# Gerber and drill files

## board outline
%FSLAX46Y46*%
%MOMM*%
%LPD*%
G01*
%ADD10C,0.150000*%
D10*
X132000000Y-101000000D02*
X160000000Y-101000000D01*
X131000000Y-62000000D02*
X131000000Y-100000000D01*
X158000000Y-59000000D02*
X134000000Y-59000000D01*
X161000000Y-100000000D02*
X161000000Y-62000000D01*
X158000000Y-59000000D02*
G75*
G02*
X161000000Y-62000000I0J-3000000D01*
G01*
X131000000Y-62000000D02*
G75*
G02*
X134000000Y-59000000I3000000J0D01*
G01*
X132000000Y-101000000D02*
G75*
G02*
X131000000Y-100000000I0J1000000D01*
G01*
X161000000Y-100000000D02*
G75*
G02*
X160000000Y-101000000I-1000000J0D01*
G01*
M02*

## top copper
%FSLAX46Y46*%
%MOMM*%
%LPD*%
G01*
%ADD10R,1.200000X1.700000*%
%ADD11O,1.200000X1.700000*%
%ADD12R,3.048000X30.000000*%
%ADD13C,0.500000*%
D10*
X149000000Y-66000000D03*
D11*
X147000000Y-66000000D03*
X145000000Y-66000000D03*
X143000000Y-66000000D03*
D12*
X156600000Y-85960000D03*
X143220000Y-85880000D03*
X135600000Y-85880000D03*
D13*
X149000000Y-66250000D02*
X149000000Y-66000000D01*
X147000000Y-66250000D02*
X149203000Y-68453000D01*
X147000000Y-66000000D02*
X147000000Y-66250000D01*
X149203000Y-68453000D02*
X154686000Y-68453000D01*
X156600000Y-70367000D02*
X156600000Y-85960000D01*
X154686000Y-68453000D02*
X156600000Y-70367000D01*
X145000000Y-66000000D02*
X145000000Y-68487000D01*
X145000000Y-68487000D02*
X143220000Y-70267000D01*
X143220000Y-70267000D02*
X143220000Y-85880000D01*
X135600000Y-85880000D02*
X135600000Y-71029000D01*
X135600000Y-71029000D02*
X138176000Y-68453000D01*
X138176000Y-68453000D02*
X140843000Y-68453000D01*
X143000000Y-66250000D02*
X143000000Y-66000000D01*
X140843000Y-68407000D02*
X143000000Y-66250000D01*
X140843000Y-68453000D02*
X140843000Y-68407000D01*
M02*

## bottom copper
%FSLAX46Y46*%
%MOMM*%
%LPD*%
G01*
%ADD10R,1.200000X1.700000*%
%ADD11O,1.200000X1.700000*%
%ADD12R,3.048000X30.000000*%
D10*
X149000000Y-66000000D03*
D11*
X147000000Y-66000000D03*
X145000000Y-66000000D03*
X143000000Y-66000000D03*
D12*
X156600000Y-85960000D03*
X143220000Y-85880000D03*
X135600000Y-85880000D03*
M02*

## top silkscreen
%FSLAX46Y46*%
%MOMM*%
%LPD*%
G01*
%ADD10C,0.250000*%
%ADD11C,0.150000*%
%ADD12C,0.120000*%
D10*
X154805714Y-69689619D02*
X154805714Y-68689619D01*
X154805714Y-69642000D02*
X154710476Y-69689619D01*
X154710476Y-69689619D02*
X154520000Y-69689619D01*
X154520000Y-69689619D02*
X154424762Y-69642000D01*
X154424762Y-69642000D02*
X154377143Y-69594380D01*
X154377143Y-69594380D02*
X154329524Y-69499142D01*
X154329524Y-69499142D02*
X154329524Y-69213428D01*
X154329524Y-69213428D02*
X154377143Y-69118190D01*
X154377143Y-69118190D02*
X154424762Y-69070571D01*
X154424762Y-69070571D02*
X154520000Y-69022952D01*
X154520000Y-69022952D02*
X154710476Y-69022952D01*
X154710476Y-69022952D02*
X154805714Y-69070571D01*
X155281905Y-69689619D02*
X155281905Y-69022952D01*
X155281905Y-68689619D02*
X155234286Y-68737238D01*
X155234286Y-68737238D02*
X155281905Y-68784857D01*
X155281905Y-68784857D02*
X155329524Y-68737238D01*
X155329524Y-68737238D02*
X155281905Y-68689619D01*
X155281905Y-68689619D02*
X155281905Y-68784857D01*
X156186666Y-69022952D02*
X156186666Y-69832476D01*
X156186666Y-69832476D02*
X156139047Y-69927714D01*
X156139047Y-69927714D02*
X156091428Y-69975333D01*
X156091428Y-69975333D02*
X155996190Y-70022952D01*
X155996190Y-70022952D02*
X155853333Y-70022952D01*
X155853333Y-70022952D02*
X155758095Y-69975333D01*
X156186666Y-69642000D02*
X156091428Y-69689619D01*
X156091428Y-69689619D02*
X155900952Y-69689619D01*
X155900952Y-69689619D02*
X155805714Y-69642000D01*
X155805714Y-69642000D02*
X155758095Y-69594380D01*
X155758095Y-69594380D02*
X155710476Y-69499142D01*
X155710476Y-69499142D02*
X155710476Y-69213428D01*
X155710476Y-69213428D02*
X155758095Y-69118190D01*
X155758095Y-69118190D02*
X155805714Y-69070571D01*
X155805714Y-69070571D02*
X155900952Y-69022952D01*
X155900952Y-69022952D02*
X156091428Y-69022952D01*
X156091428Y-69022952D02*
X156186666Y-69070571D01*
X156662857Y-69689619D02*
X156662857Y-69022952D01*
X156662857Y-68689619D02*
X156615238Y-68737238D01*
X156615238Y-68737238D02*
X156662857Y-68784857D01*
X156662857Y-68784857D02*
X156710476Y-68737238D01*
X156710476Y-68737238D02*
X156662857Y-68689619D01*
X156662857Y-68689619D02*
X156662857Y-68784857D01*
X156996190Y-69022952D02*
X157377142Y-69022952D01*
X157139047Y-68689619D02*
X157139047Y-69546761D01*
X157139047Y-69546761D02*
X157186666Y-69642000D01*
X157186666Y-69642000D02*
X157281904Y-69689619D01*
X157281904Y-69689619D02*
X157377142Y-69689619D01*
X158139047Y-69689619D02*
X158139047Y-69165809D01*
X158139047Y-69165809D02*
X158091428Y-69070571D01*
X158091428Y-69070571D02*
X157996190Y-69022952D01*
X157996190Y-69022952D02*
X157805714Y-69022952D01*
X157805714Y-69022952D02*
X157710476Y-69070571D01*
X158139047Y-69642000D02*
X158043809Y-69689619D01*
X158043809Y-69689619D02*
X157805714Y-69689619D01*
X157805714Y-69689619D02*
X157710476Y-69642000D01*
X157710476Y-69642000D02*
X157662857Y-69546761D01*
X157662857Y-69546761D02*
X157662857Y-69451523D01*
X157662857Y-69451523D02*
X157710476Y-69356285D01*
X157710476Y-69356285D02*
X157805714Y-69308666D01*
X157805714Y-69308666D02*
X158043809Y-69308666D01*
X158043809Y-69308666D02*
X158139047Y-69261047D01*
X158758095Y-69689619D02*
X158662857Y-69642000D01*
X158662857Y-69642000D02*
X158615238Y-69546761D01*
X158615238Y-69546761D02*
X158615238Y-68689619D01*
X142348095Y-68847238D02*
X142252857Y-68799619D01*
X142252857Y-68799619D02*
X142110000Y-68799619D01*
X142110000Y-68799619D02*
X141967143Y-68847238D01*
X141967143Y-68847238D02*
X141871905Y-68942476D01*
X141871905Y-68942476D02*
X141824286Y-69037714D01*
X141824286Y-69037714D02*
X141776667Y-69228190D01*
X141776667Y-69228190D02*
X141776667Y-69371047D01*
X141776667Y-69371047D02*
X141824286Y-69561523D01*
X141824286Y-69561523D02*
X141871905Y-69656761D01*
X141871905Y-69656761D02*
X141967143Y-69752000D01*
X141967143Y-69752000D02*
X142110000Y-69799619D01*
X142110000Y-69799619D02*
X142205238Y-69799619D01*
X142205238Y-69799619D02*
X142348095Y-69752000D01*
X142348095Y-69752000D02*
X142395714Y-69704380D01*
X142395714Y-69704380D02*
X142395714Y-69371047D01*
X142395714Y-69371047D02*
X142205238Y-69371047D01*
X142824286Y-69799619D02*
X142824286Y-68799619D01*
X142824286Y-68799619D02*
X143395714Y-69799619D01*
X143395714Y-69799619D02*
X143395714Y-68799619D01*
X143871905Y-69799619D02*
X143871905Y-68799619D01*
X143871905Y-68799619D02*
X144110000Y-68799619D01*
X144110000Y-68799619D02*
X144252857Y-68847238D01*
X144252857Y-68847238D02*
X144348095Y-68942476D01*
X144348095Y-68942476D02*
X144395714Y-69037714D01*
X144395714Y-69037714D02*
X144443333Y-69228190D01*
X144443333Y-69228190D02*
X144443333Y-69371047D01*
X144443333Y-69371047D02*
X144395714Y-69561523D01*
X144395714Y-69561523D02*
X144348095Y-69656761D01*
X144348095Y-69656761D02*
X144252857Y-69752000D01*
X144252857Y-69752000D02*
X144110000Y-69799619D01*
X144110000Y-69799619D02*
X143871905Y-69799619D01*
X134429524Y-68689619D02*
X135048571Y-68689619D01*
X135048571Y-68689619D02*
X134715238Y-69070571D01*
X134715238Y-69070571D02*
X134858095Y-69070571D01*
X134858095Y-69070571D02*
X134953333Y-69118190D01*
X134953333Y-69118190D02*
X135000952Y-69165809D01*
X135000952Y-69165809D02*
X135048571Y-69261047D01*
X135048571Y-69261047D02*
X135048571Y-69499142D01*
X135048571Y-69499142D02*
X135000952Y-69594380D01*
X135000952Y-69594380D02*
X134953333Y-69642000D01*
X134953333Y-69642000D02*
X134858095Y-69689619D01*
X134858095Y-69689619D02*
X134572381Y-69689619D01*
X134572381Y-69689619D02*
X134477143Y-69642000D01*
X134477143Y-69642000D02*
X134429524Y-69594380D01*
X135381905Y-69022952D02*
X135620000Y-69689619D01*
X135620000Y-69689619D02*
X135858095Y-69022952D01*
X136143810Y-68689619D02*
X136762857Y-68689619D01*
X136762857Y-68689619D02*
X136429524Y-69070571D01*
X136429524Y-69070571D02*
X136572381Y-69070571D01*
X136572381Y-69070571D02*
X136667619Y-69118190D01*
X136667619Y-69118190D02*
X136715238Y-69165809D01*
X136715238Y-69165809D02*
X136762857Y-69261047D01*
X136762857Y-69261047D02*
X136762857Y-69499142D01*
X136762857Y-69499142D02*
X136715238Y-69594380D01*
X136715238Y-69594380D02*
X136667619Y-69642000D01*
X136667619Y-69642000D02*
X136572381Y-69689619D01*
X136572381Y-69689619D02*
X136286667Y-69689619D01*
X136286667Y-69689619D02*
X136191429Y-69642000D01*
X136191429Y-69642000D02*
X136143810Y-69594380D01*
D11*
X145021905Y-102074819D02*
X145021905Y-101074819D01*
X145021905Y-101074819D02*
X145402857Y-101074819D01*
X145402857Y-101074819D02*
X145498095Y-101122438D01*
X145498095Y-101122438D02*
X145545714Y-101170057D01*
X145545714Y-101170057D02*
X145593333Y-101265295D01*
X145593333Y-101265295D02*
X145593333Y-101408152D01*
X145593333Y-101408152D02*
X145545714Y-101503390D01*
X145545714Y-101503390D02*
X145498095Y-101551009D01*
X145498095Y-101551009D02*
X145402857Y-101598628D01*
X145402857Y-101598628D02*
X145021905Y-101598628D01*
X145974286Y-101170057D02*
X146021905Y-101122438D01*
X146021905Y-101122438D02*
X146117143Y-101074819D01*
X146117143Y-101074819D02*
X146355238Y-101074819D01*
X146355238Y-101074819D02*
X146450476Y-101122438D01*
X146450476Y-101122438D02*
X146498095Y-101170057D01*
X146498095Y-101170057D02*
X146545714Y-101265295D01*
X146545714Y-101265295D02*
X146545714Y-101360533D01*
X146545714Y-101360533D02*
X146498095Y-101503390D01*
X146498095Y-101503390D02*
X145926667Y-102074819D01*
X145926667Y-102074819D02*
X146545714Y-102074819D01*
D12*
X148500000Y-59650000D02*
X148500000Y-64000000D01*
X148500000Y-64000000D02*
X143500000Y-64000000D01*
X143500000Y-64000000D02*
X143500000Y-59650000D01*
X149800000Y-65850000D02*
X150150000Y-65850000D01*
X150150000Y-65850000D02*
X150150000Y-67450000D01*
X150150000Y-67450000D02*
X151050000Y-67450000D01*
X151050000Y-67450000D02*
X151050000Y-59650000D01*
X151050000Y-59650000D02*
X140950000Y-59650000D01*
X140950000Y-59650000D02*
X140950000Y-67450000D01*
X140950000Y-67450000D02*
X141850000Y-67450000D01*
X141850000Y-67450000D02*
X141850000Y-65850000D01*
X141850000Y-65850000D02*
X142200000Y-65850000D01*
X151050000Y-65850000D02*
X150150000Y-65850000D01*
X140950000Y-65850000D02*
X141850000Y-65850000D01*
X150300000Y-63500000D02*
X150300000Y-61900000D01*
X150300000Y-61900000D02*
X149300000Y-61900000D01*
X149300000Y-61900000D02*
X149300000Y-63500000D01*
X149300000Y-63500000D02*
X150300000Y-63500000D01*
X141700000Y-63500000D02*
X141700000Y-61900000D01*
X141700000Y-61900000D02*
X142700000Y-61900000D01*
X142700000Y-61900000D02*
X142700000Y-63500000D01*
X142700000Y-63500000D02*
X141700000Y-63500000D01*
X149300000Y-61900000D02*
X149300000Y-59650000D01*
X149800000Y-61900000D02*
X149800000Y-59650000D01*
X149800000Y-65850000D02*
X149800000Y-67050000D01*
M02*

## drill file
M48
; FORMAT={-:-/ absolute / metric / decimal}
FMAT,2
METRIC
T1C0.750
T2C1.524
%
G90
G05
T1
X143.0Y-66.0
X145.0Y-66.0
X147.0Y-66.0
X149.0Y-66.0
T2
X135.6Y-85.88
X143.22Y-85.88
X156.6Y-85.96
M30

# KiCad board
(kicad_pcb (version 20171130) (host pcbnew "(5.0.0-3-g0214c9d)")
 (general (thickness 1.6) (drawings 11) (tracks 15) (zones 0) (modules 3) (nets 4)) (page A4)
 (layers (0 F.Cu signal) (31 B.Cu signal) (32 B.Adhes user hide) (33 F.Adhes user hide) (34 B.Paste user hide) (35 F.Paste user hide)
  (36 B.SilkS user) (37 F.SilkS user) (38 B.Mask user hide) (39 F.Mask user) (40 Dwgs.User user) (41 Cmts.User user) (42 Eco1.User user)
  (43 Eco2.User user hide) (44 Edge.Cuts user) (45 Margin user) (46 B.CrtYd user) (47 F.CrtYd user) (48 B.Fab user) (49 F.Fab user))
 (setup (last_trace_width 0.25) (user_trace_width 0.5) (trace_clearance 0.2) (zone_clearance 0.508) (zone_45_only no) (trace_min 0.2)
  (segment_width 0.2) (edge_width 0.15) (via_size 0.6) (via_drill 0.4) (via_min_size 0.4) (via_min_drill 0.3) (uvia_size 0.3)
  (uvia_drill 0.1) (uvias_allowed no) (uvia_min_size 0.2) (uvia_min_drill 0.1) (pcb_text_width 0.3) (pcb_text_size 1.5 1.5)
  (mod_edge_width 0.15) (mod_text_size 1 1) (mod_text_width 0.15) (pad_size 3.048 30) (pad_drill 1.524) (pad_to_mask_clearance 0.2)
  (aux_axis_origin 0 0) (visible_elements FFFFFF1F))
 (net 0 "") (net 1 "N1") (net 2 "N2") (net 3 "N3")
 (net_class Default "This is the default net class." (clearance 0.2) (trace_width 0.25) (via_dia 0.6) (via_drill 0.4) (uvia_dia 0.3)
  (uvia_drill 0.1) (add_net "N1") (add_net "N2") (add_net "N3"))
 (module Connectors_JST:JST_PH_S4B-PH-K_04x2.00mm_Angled (layer F.Cu) (at 149 66 180)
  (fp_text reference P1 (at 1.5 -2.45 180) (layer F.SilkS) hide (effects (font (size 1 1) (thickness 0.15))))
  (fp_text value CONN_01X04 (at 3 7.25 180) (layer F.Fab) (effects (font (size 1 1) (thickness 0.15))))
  (fp_line (start 0.5 6.35) (end 0.5 2) (layer F.SilkS) (width 0.12))
  (fp_line (start 0.5 2) (end 5.5 2) (layer F.SilkS) (width 0.12))
  (fp_line (start 5.5 2) (end 5.5 6.35) (layer F.SilkS) (width 0.12))
  (fp_line (start -0.8 0.15) (end -1.15 0.15) (layer F.SilkS) (width 0.12))
  (fp_line (start -1.15 0.15) (end -1.15 -1.45) (layer F.SilkS) (width 0.12))
  (fp_line (start -1.15 -1.45) (end -2.05 -1.45) (layer F.SilkS) (width 0.12))
  (fp_line (start -2.05 -1.45) (end -2.05 6.35) (layer F.SilkS) (width 0.12))
  (fp_line (start -2.05 6.35) (end 8.05 6.35) (layer F.SilkS) (width 0.12))
  (fp_line (start 8.05 6.35) (end 8.05 -1.45) (layer F.SilkS) (width 0.12))
  (fp_line (start 8.05 -1.45) (end 7.15 -1.45) (layer F.SilkS) (width 0.12))
  (fp_line (start 7.15 -1.45) (end 7.15 0.15) (layer F.SilkS) (width 0.12))
  (fp_line (start 7.15 0.15) (end 6.8 0.15) (layer F.SilkS) (width 0.12))
  (fp_line (start -2.05 0.15) (end -1.15 0.15) (layer F.SilkS) (width 0.12))
  (fp_line (start 8.05 0.15) (end 7.15 0.15) (layer F.SilkS) (width 0.12))
  (fp_line (start -1.3 2.5) (end -1.3 4.1) (layer F.SilkS) (width 0.12))
  (fp_line (start -1.3 4.1) (end -0.3 4.1) (layer F.SilkS) (width 0.12))
  (fp_line (start -0.3 4.1) (end -0.3 2.5) (layer F.SilkS) (width 0.12))
  (fp_line (start -0.3 2.5) (end -1.3 2.5) (layer F.SilkS) (width 0.12))
  (fp_line (start 7.3 2.5) (end 7.3 4.1) (layer F.SilkS) (width 0.12))
  (fp_line (start 7.3 4.1) (end 6.3 4.1) (layer F.SilkS) (width 0.12))
  (fp_line (start 6.3 4.1) (end 6.3 2.5) (layer F.SilkS) (width 0.12))
  (fp_line (start 6.3 2.5) (end 7.3 2.5) (layer F.SilkS) (width 0.12))
  (fp_line (start -0.3 4.1) (end -0.3 6.35) (layer F.SilkS) (width 0.12))
  (fp_line (start -0.8 4.1) (end -0.8 6.35) (layer F.SilkS) (width 0.12))
  (fp_line (start -0.8 0.15) (end -0.8 -1.05) (layer F.SilkS) (width 0.12))
  (pad 1 thru_hole rect (at 0 0 180) (size 1.2 1.7) (drill 0.75) (layers *.Cu *.Mask))
  (pad 2 thru_hole oval (at 2 0 180) (size 1.2 1.7) (drill 0.75) (layers *.Cu *.Mask) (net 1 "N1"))
  (pad 3 thru_hole oval (at 4 0 180) (size 1.2 1.7) (drill 0.75) (layers *.Cu *.Mask) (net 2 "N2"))
  (pad 4 thru_hole oval (at 6 0 180) (size 1.2 1.7) (drill 0.75) (layers *.Cu *.Mask) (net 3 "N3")))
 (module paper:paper (layer F.Cu) (at 145.76 101.12)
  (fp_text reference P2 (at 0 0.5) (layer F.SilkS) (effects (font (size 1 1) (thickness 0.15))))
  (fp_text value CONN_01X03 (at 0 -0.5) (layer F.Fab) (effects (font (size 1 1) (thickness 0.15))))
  (pad 3 thru_hole rect (at 10.84 -15.16) (size 3.048 30) (drill 1.524) (layers *.Cu *.Mask) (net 1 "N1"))
  (pad 2 thru_hole rect (at -2.54 -15.24) (size 3.048 30) (drill 1.524) (layers *.Cu *.Mask) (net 2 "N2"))
  (pad 1 thru_hole rect (at -10.16 -15.24) (size 3.048 30) (drill 1.524) (layers *.Cu *.Mask) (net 3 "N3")))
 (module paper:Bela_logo (layer B.Cu) (at 155.067 64.897 135)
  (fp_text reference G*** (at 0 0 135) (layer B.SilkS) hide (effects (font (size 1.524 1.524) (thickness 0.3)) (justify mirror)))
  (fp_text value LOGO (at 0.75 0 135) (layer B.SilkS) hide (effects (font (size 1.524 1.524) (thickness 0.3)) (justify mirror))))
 (gr_line (start 132 101) (end 160 101) (angle 90) (layer Edge.Cuts) (width 0.15))
 (gr_line (start 131 62) (end 131 100) (angle 90) (layer Edge.Cuts) (width 0.15))
 (gr_line (start 158 59) (end 134 59) (angle 90) (layer Edge.Cuts) (width 0.15))
 (gr_line (start 161 100) (end 161 62) (angle 90) (layer Edge.Cuts) (width 0.15))
 (gr_arc (start 158 62) (end 158 59) (angle 90) (layer Edge.Cuts) (width 0.15))
 (gr_arc (start 134 62) (end 131 62) (angle 90) (layer Edge.Cuts) (width 0.15))
 (gr_arc (start 132 100) (end 132 101) (angle 90) (layer Edge.Cuts) (width 0.15))
 (gr_arc (start 160 100) (end 161 100) (angle 90) (layer Edge.Cuts) (width 0.15))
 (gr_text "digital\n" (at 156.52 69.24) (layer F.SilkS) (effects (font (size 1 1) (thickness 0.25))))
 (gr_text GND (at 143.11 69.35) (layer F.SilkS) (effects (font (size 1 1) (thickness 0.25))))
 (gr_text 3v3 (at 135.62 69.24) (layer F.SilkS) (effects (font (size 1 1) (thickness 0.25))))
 (segment (start 149 66.25) (end 149 66) (width 0.5) (layer F.Cu) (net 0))
 (segment (start 147 66.25) (end 149.203 68.453) (width 0.5) (layer F.Cu) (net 1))
 (segment (start 147 66) (end 147 66.25) (width 0.5) (layer F.Cu) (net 1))
 (segment (start 149.203 68.453) (end 154.686 68.453) (width 0.5) (layer F.Cu) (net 1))
 (segment (start 156.6 70.367) (end 156.6 85.96) (width 0.5) (layer F.Cu) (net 1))
 (segment (start 154.686 68.453) (end 156.6 70.367) (width 0.5) (layer F.Cu) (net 1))
 (segment (start 145 66) (end 145 68.487) (width 0.5) (layer F.Cu) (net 2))
 (segment (start 145 68.487) (end 143.22 70.267) (width 0.5) (layer F.Cu) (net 2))
 (segment (start 143.22 70.267) (end 143.22 85.88) (width 0.5) (layer F.Cu) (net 2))
 (segment (start 135.6 85.88) (end 135.6 71.029) (width 0.5) (layer F.Cu) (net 3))
 (segment (start 135.6 71.029) (end 138.176 68.453) (width 0.5) (layer F.Cu) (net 3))
 (segment (start 138.176 68.453) (end 140.843 68.453) (width 0.5) (layer F.Cu) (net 3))
 (segment (start 143 66.25) (end 143 66) (width 0.5) (layer F.Cu) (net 3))
 (segment (start 140.843 68.407) (end 143 66.25) (width 0.5) (layer F.Cu) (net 3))
 (segment (start 140.843 68.453) (end 140.843 68.407) (width 0.5) (layer F.Cu) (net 3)))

